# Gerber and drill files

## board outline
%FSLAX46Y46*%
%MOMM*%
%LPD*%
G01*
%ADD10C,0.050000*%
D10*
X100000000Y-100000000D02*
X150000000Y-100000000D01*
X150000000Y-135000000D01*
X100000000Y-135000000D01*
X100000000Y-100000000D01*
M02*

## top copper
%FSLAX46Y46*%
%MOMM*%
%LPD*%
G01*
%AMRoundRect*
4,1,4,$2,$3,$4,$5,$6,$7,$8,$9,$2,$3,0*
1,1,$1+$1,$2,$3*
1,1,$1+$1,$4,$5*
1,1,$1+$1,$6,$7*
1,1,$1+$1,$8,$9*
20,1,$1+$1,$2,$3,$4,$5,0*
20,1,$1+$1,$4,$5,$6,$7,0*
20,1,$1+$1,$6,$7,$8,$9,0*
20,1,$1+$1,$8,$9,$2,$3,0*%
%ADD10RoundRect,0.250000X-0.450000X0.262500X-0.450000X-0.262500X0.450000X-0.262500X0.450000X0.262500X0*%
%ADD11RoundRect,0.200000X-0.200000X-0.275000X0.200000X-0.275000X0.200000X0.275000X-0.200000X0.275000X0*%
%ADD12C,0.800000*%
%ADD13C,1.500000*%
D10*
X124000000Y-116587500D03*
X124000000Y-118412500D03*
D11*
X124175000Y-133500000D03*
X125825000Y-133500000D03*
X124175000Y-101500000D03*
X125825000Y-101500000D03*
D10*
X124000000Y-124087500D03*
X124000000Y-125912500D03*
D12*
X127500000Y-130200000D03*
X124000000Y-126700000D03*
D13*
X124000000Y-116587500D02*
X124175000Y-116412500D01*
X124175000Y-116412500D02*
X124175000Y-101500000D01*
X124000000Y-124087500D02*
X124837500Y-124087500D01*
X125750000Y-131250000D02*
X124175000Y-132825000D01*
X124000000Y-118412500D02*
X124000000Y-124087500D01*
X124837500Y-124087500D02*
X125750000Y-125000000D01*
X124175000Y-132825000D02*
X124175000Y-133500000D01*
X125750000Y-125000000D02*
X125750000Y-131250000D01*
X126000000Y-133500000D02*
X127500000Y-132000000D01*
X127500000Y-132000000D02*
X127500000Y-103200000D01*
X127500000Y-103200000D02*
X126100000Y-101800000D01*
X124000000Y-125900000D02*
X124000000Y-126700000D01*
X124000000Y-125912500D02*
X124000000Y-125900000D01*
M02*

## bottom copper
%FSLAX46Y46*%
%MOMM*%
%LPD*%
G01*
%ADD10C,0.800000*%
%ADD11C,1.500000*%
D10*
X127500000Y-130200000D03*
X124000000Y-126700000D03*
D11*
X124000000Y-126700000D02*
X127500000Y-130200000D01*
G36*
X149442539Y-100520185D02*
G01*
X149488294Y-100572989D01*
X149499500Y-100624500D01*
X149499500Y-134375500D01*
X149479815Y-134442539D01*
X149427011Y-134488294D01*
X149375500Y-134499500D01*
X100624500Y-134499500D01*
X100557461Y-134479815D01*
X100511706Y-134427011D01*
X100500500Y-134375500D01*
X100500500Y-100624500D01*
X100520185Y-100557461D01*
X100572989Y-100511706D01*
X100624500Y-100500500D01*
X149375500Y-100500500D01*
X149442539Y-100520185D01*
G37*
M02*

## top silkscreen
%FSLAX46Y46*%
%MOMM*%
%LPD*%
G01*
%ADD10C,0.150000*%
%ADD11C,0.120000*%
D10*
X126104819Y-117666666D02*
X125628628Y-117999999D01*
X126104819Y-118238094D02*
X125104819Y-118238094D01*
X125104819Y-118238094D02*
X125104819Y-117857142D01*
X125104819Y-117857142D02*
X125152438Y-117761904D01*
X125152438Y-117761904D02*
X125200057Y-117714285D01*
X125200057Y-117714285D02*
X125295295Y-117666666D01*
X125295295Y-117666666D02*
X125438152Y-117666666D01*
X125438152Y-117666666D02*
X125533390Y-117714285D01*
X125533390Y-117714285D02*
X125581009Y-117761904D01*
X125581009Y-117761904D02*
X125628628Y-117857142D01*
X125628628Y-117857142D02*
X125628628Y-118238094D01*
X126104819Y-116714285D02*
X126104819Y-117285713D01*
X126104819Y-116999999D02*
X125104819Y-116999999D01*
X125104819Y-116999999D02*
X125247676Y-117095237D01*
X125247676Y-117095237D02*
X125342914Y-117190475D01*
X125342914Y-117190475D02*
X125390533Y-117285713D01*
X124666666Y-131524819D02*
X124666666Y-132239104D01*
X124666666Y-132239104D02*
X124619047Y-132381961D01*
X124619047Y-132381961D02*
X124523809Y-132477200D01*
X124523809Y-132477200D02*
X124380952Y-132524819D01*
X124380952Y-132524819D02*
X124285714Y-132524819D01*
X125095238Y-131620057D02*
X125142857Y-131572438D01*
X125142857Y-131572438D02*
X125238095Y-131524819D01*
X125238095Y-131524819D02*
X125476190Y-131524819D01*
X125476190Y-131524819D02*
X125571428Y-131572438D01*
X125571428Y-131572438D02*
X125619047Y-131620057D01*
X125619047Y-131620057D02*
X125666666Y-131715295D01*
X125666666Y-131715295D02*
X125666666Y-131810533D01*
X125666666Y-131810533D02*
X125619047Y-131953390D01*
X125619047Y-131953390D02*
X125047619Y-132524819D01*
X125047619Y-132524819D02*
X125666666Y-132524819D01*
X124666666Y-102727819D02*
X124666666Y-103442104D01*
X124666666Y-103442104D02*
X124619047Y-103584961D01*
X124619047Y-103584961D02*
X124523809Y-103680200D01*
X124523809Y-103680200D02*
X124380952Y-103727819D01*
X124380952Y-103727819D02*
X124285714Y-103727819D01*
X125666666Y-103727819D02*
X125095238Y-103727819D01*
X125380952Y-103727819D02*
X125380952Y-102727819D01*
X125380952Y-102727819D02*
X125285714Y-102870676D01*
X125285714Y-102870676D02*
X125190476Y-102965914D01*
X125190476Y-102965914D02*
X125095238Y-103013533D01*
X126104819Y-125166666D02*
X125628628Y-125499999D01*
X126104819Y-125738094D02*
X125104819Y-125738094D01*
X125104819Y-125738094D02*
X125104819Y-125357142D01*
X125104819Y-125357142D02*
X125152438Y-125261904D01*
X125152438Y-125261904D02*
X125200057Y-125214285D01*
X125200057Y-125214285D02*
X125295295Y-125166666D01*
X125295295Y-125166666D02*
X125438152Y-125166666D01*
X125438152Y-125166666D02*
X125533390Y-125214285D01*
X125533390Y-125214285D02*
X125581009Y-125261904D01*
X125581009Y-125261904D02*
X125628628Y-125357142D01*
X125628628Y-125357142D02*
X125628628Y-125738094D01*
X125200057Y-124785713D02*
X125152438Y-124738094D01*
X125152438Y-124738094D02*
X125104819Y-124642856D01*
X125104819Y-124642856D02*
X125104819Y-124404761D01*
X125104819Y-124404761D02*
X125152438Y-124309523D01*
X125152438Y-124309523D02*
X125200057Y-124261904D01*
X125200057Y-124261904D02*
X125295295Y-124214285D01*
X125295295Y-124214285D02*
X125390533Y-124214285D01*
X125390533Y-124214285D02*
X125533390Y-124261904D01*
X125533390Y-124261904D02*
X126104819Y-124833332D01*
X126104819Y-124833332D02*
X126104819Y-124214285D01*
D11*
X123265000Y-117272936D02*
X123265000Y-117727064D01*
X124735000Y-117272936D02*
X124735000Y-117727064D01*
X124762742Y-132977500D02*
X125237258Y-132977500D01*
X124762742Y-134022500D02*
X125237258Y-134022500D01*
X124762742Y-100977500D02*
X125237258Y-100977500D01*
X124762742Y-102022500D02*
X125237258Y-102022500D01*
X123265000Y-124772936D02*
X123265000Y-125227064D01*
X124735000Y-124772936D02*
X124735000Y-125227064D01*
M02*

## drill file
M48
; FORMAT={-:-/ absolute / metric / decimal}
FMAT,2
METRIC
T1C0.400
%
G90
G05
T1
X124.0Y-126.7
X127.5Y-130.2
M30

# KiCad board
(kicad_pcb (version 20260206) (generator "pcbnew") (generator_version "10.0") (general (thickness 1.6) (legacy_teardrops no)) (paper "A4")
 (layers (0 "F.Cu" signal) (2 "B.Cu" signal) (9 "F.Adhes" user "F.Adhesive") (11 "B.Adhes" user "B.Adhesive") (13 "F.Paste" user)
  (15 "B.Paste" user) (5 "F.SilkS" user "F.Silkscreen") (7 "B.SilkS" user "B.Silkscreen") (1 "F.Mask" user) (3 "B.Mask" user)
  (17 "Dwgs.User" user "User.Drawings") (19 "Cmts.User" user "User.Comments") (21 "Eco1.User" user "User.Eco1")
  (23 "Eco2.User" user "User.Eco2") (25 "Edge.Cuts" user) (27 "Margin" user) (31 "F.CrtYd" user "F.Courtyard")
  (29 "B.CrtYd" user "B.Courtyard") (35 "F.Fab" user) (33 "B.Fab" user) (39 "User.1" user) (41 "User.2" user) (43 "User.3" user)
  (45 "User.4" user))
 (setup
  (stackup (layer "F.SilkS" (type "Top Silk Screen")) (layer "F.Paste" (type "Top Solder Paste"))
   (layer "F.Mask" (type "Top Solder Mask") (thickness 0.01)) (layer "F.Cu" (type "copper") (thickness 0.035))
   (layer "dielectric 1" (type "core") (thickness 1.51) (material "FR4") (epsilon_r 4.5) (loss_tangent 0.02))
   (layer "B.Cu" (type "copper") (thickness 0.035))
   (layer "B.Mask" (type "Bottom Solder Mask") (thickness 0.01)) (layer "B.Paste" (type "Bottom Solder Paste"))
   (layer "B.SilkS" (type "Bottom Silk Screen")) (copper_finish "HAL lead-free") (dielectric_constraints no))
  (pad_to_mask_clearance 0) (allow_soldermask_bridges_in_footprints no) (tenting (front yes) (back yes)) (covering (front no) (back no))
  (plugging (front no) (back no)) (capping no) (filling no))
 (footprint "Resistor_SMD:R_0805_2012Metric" (layer "F.Cu") (at 124 117.5 -90)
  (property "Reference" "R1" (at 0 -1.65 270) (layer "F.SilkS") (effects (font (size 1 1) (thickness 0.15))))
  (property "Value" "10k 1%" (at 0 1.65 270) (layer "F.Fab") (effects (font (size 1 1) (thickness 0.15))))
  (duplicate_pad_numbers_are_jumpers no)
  (fp_line (start -0.227064 0.735) (end 0.227064 0.735) (stroke (width 0.12) (type solid)) (layer "F.SilkS"))
  (fp_line (start -0.227064 -0.735) (end 0.227064 -0.735) (stroke (width 0.12) (type solid)) (layer "F.SilkS"))
  (pad "1" smd roundrect (at -0.9125 0 270) (size 1.025 1.4) (layers "F.Cu" "F.Mask" "F.Paste") (roundrect_rratio 0.243902) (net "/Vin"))
  (pad "2" smd roundrect (at 0.9125 0 270) (size 1.025 1.4) (layers "F.Cu" "F.Mask" "F.Paste") (roundrect_rratio 0.243902) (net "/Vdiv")))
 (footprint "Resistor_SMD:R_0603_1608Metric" (layer "F.Cu") (at 125 133.5)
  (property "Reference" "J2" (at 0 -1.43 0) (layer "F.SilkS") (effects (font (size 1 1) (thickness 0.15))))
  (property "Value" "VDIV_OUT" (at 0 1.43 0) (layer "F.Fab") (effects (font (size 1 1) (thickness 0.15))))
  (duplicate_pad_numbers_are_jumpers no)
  (fp_line (start -0.237258 -0.5225) (end 0.237258 -0.5225) (stroke (width 0.12) (type solid)) (layer "F.SilkS"))
  (fp_line (start -0.237258 0.5225) (end 0.237258 0.5225) (stroke (width 0.12) (type solid)) (layer "F.SilkS"))
  (pad "1" smd roundrect (at -0.825 0) (size 0.8 0.95) (layers "F.Cu" "F.Mask" "F.Paste") (roundrect_rratio 0.25) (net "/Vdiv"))
  (pad "2" smd roundrect (at 0.825 0) (size 0.8 0.95) (layers "F.Cu" "F.Mask" "F.Paste") (roundrect_rratio 0.25) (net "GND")))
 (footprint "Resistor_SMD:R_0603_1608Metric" (layer "F.Cu") (at 125 101.5)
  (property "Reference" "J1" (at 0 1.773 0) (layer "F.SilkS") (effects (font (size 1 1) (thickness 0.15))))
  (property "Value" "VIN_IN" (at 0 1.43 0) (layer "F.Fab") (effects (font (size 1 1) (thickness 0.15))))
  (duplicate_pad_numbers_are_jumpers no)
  (fp_line (start -0.237258 -0.5225) (end 0.237258 -0.5225) (stroke (width 0.12) (type solid)) (layer "F.SilkS"))
  (fp_line (start -0.237258 0.5225) (end 0.237258 0.5225) (stroke (width 0.12) (type solid)) (layer "F.SilkS"))
  (pad "1" smd roundrect (at -0.825 0) (size 0.8 0.95) (layers "F.Cu" "F.Mask" "F.Paste") (roundrect_rratio 0.25) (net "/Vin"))
  (pad "2" smd roundrect (at 0.825 0) (size 0.8 0.95) (layers "F.Cu" "F.Mask" "F.Paste") (roundrect_rratio 0.25) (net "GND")))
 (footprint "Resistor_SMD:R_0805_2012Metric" (layer "F.Cu") (at 124 125 -90)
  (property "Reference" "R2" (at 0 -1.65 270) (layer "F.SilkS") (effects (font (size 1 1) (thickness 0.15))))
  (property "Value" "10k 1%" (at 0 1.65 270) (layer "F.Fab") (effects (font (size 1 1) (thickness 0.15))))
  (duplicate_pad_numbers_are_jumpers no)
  (fp_line (start -0.227064 0.735) (end 0.227064 0.735) (stroke (width 0.12) (type solid)) (layer "F.SilkS"))
  (fp_line (start -0.227064 -0.735) (end 0.227064 -0.735) (stroke (width 0.12) (type solid)) (layer "F.SilkS"))
  (pad "1" smd roundrect (at -0.9125 0 270) (size 1.025 1.4) (layers "F.Cu" "F.Mask" "F.Paste") (roundrect_rratio 0.243902) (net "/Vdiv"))
  (pad "2" smd roundrect (at 0.9125 0 270) (size 1.025 1.4) (layers "F.Cu" "F.Mask" "F.Paste") (roundrect_rratio 0.243902) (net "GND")))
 (gr_rect (start 100 100) (end 150 135) (stroke (width 0.05) (type solid)) (fill no) (layer "Edge.Cuts"))
 (segment (start 124 116.5875) (end 124.175 116.4125) (width 1.5) (layer "F.Cu") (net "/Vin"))
 (segment (start 124.175 116.4125) (end 124.175 101.5) (width 1.5) (layer "F.Cu") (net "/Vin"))
 (segment (start 124 124.0875) (end 124.8375 124.0875) (width 1.5) (layer "F.Cu") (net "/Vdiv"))
 (segment (start 125.75 131.25) (end 124.175 132.825) (width 1.5) (layer "F.Cu") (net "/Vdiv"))
 (segment (start 124 118.4125) (end 124 124.0875) (width 1.5) (layer "F.Cu") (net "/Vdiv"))
 (segment (start 124.8375 124.0875) (end 125.75 125) (width 1.5) (layer "F.Cu") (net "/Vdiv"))
 (segment (start 124.175 132.825) (end 124.175 133.5) (width 1.5) (layer "F.Cu") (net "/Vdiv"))
 (segment (start 125.75 125) (end 125.75 131.25) (width 1.5) (layer "F.Cu") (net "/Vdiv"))
 (segment (start 126 133.5) (end 127.5 132) (width 1.5) (layer "F.Cu") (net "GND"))
 (segment (start 127.5 132) (end 127.5 103.2) (width 1.5) (layer "F.Cu") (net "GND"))
 (segment (start 127.5 103.2) (end 126.1 101.8) (width 1.5) (layer "F.Cu") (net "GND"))
 (segment (start 124 125.9) (end 124 126.7) (width 1.5) (layer "F.Cu") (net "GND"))
 (segment (start 124 125.9125) (end 124 125.9) (width 1.5) (layer "F.Cu") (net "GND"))
 (via (at 127.5 130.2) (size 0.8) (drill 0.4) (layers "F.Cu" "B.Cu") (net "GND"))
 (via (at 124 126.7) (size 0.8) (drill 0.4) (layers "F.Cu" "B.Cu") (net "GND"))
 (segment (start 124 126.7) (end 127.5 130.2) (width 1.5) (layer "B.Cu") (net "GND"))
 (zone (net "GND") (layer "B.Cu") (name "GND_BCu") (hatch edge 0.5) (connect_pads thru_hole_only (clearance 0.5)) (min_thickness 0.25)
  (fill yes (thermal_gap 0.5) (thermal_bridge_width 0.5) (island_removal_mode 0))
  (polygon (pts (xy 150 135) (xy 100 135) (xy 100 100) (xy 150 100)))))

